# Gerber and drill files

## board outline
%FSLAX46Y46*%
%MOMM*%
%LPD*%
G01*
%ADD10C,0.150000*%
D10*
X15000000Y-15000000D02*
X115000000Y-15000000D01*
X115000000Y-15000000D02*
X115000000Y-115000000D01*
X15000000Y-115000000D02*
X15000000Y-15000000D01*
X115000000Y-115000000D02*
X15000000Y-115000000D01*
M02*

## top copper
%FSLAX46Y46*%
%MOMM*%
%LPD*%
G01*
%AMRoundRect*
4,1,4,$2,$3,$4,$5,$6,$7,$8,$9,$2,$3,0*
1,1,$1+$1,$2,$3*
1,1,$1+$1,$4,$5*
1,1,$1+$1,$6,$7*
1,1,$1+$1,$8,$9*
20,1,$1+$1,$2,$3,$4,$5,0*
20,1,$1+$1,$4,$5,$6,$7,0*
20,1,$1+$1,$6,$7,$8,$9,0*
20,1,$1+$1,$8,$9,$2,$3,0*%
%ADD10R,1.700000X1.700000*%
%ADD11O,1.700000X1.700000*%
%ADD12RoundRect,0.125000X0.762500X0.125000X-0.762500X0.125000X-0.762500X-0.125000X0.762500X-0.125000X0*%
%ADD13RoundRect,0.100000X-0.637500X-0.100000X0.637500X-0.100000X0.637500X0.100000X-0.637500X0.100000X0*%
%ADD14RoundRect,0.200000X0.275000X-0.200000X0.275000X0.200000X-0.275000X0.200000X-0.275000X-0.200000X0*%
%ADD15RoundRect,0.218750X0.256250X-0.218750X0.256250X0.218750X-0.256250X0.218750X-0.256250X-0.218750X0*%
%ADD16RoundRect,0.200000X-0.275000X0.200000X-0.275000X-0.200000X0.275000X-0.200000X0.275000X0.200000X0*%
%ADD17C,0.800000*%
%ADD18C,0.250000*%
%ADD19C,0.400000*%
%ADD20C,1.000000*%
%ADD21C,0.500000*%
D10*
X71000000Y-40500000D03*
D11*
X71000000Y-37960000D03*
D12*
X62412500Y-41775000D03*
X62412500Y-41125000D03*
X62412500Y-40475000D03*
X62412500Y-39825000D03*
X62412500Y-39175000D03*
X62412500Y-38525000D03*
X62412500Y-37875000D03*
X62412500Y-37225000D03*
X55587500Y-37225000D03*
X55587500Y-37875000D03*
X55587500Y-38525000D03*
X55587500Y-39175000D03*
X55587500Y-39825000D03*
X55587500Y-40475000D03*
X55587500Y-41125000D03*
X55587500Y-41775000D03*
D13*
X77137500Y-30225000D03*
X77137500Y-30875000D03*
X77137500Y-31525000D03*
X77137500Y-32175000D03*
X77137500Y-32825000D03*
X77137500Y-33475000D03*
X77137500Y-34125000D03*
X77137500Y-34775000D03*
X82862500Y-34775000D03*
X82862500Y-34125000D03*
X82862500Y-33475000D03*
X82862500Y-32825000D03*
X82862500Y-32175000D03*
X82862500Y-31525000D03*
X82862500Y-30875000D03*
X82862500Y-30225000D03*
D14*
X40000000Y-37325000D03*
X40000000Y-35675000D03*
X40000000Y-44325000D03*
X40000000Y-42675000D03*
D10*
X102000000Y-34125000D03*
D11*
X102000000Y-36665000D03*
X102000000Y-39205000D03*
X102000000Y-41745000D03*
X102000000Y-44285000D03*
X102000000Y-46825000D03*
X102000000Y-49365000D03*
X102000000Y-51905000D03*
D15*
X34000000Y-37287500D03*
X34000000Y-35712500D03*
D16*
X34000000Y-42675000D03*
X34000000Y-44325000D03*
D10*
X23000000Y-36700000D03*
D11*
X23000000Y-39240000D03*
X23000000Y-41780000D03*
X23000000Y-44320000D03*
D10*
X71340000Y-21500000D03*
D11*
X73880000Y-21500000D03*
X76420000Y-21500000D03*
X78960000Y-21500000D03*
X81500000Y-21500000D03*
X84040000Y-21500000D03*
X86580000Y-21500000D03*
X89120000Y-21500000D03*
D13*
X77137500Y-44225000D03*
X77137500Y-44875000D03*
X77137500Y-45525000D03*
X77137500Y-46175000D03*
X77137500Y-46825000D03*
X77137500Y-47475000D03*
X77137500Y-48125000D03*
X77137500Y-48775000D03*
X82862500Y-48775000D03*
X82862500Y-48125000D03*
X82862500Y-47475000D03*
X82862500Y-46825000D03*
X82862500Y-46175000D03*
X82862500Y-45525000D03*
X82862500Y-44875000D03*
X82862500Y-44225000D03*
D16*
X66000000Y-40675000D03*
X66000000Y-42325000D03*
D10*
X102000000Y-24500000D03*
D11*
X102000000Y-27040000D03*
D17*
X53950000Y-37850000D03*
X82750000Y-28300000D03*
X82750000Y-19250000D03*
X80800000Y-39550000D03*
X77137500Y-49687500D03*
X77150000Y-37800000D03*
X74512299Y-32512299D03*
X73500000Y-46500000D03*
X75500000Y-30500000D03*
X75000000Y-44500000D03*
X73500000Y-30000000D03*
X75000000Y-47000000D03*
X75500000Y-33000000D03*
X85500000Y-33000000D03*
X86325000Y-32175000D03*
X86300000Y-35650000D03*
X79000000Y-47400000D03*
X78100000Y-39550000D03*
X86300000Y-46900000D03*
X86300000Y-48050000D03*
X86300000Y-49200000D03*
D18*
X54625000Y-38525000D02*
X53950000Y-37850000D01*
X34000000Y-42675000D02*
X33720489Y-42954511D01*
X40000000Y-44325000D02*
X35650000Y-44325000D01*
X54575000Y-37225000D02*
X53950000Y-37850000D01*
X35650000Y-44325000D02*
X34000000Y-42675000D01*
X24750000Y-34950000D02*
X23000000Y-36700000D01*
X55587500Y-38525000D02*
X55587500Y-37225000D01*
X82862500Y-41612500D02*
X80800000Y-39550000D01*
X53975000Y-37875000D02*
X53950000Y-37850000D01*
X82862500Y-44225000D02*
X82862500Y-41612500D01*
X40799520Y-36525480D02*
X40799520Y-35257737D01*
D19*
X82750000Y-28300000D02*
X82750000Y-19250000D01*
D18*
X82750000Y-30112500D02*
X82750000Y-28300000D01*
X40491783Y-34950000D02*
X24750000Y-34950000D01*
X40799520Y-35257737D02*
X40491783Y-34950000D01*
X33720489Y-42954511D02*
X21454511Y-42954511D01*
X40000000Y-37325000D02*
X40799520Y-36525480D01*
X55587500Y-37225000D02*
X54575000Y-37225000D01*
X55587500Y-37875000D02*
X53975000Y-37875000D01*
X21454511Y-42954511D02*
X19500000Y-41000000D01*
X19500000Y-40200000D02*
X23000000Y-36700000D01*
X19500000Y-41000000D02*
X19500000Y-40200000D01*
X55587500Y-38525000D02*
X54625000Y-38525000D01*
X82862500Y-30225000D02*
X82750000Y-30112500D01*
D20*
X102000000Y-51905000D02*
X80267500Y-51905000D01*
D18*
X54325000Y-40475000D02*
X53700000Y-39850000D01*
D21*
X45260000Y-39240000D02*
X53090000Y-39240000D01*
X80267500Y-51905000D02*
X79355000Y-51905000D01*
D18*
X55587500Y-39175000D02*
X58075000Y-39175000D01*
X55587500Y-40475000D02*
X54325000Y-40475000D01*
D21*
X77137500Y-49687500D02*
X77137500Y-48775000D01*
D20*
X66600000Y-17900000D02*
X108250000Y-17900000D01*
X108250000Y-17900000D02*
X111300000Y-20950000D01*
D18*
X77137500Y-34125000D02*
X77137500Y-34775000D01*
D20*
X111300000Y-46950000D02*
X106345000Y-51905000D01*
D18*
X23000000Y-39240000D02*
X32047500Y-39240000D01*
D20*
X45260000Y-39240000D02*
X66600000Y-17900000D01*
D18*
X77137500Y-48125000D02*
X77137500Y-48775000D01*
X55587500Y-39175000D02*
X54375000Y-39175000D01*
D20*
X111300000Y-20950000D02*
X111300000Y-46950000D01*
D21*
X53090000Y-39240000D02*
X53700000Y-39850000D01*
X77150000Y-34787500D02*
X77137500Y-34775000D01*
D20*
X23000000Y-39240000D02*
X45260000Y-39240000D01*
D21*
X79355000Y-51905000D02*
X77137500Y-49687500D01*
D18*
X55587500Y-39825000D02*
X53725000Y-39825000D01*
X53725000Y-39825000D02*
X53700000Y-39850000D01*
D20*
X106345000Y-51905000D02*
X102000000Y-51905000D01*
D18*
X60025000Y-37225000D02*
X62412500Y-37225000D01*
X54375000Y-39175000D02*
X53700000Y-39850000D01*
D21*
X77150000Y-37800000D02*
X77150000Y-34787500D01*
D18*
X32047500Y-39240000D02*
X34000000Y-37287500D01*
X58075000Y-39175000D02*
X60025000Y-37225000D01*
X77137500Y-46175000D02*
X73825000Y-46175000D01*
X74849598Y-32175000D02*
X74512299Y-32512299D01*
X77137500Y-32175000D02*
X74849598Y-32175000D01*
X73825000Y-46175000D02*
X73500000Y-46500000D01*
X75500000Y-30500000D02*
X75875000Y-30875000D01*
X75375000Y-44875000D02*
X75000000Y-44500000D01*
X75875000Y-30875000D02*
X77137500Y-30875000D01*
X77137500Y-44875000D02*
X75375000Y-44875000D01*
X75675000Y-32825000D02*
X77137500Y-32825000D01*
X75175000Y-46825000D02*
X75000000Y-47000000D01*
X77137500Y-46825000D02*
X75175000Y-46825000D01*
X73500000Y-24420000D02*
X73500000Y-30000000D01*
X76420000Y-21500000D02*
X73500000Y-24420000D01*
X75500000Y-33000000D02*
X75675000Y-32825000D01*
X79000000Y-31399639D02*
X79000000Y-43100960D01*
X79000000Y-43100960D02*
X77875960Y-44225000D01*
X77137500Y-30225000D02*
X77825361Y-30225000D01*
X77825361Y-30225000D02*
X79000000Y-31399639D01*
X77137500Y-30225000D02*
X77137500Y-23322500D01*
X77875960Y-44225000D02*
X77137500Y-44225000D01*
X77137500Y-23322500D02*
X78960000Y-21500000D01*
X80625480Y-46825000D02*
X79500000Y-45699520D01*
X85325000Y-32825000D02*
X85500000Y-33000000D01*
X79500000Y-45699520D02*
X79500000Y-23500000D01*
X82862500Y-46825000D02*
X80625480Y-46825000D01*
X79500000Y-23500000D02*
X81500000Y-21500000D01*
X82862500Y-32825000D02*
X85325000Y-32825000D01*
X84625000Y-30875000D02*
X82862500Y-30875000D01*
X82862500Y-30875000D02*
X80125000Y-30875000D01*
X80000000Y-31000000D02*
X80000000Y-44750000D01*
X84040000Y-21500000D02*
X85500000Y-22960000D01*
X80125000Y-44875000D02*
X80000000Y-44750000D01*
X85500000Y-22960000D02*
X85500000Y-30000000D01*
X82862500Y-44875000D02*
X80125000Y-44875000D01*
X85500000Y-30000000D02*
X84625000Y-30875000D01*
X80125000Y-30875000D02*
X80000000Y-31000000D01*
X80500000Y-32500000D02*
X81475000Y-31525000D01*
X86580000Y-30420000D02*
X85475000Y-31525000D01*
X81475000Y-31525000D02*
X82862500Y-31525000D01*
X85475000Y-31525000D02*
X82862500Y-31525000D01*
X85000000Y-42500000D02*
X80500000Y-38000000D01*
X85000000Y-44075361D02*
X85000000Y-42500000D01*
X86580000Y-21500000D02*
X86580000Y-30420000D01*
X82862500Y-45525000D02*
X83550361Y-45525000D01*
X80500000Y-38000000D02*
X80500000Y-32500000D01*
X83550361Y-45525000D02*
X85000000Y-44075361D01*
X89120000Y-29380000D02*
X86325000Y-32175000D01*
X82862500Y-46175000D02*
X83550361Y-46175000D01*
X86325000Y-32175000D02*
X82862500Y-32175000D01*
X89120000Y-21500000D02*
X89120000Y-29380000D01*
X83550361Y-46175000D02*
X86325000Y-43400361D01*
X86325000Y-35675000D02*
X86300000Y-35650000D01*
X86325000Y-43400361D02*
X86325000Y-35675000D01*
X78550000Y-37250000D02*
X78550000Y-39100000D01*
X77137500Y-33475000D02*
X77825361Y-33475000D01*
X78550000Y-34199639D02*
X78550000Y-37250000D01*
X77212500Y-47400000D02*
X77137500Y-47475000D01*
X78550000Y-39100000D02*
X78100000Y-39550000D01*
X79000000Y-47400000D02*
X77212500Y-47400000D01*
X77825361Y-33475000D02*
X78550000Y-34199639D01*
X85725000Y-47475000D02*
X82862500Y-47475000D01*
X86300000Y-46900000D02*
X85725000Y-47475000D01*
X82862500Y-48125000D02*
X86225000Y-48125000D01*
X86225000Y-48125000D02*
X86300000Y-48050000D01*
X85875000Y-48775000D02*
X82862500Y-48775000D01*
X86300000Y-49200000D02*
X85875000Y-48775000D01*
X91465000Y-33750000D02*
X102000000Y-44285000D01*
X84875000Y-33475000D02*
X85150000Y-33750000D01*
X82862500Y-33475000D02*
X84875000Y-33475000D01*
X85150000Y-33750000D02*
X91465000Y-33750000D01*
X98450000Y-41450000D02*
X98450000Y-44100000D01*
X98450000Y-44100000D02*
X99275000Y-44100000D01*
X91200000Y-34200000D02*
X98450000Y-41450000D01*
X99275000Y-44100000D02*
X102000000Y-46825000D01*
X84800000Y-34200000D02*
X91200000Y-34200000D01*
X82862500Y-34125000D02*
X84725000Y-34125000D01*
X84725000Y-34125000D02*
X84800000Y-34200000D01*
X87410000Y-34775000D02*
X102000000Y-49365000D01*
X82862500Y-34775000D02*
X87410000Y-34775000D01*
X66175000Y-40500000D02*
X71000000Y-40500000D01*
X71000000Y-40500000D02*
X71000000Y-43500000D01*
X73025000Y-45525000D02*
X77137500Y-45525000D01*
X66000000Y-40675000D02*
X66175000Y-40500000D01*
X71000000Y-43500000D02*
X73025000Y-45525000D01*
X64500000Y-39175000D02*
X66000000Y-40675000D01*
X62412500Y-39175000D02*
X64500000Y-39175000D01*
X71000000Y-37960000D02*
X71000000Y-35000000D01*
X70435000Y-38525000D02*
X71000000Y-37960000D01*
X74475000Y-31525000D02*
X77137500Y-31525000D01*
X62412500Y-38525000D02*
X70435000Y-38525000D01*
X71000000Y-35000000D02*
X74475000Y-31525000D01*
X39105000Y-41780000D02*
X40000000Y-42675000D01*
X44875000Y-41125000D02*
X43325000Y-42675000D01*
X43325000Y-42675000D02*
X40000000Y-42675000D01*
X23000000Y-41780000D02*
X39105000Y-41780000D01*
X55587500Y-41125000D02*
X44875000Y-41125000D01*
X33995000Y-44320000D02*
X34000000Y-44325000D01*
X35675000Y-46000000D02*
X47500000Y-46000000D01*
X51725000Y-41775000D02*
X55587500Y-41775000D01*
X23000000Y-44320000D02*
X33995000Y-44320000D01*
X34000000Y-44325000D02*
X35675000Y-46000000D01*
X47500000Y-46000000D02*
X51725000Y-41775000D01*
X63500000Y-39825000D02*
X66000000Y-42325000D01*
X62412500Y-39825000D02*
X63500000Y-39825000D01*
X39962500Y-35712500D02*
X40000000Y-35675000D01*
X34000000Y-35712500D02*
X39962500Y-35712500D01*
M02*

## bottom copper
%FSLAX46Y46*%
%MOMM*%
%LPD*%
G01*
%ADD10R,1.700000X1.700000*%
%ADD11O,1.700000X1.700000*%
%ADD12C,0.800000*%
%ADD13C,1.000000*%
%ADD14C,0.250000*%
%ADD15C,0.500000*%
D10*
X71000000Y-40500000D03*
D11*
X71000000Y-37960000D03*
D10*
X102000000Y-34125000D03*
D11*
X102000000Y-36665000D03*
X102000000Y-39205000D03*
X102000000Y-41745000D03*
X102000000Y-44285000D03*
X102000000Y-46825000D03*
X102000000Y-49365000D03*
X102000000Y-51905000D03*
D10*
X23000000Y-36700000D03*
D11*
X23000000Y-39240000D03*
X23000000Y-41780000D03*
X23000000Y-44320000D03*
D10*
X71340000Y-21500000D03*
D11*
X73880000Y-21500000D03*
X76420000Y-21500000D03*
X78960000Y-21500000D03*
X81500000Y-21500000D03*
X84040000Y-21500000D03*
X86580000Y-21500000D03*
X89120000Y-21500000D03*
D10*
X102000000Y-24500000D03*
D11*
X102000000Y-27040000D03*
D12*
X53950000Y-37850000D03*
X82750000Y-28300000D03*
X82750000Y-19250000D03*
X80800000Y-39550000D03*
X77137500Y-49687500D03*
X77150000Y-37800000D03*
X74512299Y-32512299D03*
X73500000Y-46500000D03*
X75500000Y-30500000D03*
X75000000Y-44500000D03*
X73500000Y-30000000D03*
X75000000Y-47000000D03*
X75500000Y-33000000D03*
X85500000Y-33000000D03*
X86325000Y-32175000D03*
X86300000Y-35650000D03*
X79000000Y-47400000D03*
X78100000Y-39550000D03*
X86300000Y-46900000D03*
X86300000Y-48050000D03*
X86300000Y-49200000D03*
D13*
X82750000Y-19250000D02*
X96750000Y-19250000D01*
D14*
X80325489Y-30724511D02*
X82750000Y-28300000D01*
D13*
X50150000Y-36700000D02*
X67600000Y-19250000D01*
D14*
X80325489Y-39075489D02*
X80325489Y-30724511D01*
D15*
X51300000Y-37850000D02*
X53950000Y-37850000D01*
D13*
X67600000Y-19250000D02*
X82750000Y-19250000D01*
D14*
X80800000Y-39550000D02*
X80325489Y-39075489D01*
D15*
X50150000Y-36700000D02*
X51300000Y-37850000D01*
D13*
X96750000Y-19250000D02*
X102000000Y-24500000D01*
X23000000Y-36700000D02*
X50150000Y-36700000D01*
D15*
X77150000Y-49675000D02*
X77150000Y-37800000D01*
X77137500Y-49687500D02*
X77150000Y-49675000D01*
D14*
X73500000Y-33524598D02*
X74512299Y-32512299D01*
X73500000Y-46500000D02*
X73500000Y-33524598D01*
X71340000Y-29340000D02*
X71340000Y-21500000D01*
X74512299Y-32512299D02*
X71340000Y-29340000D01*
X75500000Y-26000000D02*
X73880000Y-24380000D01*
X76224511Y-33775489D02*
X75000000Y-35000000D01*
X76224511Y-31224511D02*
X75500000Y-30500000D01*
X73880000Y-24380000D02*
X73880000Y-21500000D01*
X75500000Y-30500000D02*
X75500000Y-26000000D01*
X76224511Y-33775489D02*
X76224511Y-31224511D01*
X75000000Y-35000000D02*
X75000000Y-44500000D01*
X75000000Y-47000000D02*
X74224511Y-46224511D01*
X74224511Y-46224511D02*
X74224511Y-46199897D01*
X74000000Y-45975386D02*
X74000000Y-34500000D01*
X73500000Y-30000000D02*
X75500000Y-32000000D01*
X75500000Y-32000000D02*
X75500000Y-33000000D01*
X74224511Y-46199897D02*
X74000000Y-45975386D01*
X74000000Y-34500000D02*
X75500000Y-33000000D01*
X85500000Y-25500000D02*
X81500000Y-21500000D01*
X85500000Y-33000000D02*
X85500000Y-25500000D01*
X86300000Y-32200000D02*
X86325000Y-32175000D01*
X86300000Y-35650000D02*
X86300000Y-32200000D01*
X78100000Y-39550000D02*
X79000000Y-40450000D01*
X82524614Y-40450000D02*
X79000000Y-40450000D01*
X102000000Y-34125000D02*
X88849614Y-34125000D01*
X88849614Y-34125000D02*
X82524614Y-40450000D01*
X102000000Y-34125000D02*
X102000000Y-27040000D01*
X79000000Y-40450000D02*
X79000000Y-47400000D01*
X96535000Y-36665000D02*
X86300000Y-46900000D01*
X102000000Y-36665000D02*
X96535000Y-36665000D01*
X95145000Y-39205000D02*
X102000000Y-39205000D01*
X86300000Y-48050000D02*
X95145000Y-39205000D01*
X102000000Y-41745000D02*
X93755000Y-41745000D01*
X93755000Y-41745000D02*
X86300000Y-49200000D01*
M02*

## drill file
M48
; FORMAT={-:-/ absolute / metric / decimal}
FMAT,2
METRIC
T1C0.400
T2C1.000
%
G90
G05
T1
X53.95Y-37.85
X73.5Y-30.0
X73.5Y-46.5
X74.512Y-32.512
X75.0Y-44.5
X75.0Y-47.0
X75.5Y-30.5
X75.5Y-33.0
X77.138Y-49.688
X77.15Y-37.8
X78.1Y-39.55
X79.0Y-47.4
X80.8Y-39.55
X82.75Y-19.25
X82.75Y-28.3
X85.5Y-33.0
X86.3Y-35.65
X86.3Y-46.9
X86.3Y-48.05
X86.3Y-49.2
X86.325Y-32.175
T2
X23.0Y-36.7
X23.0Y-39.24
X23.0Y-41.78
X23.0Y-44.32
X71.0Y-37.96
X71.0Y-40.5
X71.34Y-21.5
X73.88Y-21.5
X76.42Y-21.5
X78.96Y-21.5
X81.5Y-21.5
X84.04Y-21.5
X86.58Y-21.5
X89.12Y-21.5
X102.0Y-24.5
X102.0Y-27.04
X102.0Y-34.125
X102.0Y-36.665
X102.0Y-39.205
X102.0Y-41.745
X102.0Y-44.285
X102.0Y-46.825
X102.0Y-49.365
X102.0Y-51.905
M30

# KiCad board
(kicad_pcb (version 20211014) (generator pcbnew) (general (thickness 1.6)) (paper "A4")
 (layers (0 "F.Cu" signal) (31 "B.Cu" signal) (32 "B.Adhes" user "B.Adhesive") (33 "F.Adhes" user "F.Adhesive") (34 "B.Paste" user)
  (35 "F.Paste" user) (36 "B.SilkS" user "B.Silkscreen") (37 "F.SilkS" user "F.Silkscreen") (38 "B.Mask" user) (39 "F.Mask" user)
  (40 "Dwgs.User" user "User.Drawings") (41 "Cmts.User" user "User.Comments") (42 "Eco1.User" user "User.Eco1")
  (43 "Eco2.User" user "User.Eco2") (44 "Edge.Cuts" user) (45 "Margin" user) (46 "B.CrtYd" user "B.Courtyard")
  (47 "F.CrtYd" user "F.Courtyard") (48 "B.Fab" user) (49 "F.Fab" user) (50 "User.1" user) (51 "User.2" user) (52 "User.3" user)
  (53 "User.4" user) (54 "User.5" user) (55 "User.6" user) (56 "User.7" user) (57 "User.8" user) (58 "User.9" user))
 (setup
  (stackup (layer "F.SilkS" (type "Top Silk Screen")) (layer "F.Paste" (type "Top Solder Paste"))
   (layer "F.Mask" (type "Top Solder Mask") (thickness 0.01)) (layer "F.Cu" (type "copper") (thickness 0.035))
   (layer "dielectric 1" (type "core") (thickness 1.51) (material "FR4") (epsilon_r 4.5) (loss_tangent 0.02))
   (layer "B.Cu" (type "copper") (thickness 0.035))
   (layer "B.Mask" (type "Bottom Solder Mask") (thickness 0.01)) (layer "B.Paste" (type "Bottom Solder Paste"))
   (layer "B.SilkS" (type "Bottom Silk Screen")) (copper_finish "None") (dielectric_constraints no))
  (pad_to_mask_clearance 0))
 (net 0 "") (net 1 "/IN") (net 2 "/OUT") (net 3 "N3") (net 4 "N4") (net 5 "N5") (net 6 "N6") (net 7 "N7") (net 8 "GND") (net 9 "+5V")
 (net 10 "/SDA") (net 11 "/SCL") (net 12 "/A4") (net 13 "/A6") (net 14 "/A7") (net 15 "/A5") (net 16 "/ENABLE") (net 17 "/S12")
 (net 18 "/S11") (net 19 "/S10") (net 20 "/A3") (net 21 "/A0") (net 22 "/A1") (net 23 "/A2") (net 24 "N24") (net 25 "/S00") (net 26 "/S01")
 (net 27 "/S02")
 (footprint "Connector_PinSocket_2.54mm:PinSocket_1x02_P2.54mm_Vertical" (layer "F.Cu") (at 71 40.5 180)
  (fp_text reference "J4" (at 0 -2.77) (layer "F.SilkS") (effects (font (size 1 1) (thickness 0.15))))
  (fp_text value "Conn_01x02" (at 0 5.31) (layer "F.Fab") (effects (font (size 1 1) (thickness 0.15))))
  (pad "1" thru_hole rect locked (at 0 0 180) (size 1.7 1.7) (drill 1) (layers *.Cu *.Mask) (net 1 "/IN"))
  (pad "2" thru_hole oval locked (at 0 2.54 180) (size 1.7 1.7) (drill 1) (layers *.Cu *.Mask) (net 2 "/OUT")))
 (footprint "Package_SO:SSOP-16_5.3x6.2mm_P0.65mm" (layer "F.Cu") (at 59 39.5 180)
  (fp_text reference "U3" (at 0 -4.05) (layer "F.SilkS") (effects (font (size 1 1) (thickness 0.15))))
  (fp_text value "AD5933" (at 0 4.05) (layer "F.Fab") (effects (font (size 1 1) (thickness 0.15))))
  (pad "1" smd roundrect locked (at -3.4125 -2.275 180) (size 1.775 0.5) (layers "F.Cu" "F.Paste" "F.Mask") (roundrect_rratio 0.25)
   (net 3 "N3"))
  (pad "2" smd roundrect locked (at -3.4125 -1.625 180) (size 1.775 0.5) (layers "F.Cu" "F.Paste" "F.Mask") (roundrect_rratio 0.25)
   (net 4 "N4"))
  (pad "3" smd roundrect locked (at -3.4125 -0.975 180) (size 1.775 0.5) (layers "F.Cu" "F.Paste" "F.Mask") (roundrect_rratio 0.25)
   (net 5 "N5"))
  (pad "4" smd roundrect locked (at -3.4125 -0.325 180) (size 1.775 0.5) (layers "F.Cu" "F.Paste" "F.Mask") (roundrect_rratio 0.25)
   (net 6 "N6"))
  (pad "5" smd roundrect locked (at -3.4125 0.325 180) (size 1.775 0.5) (layers "F.Cu" "F.Paste" "F.Mask") (roundrect_rratio 0.25)
   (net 1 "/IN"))
  (pad "6" smd roundrect locked (at -3.4125 0.975 180) (size 1.775 0.5) (layers "F.Cu" "F.Paste" "F.Mask") (roundrect_rratio 0.25)
   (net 2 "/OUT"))
  (pad "7" smd roundrect locked (at -3.4125 1.625 180) (size 1.775 0.5) (layers "F.Cu" "F.Paste" "F.Mask") (roundrect_rratio 0.25)
   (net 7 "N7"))
  (pad "8" smd roundrect locked (at -3.4125 2.275 180) (size 1.775 0.5) (layers "F.Cu" "F.Paste" "F.Mask") (roundrect_rratio 0.25)
   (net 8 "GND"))
  (pad "9" smd roundrect locked (at 3.4125 2.275 180) (size 1.775 0.5) (layers "F.Cu" "F.Paste" "F.Mask") (roundrect_rratio 0.25)
   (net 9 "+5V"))
  (pad "10" smd roundrect locked (at 3.4125 1.625 180) (size 1.775 0.5) (layers "F.Cu" "F.Paste" "F.Mask") (roundrect_rratio 0.25)
   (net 9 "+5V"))
  (pad "11" smd roundrect locked (at 3.4125 0.975 180) (size 1.775 0.5) (layers "F.Cu" "F.Paste" "F.Mask") (roundrect_rratio 0.25)
   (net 9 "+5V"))
  (pad "12" smd roundrect locked (at 3.4125 0.325 180) (size 1.775 0.5) (layers "F.Cu" "F.Paste" "F.Mask") (roundrect_rratio 0.25)
   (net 8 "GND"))
  (pad "13" smd roundrect locked (at 3.4125 -0.325 180) (size 1.775 0.5) (layers "F.Cu" "F.Paste" "F.Mask") (roundrect_rratio 0.25)
   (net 8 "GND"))
  (pad "14" smd roundrect locked (at 3.4125 -0.975 180) (size 1.775 0.5) (layers "F.Cu" "F.Paste" "F.Mask") (roundrect_rratio 0.25)
   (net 8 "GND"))
  (pad "15" smd roundrect locked (at 3.4125 -1.625 180) (size 1.775 0.5) (layers "F.Cu" "F.Paste" "F.Mask") (roundrect_rratio 0.25)
   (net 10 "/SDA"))
  (pad "16" smd roundrect locked (at 3.4125 -2.275 180) (size 1.775 0.5) (layers "F.Cu" "F.Paste" "F.Mask") (roundrect_rratio 0.25)
   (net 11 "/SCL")))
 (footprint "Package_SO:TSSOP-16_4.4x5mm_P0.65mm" (layer "F.Cu") (at 80 32.5)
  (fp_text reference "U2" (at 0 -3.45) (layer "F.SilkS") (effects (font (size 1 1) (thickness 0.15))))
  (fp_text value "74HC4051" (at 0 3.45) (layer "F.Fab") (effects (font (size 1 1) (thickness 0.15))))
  (pad "1" smd roundrect locked (at -2.8625 -2.275) (size 1.475 0.4) (layers "F.Cu" "F.Paste" "F.Mask") (roundrect_rratio 0.25)
   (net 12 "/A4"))
  (pad "2" smd roundrect locked (at -2.8625 -1.625) (size 1.475 0.4) (layers "F.Cu" "F.Paste" "F.Mask") (roundrect_rratio 0.25)
   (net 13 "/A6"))
  (pad "3" smd roundrect locked (at -2.8625 -0.975) (size 1.475 0.4) (layers "F.Cu" "F.Paste" "F.Mask") (roundrect_rratio 0.25)
   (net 2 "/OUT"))
  (pad "4" smd roundrect locked (at -2.8625 -0.325) (size 1.475 0.4) (layers "F.Cu" "F.Paste" "F.Mask") (roundrect_rratio 0.25)
   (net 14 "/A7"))
  (pad "5" smd roundrect locked (at -2.8625 0.325) (size 1.475 0.4) (layers "F.Cu" "F.Paste" "F.Mask") (roundrect_rratio 0.25)
   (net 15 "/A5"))
  (pad "6" smd roundrect locked (at -2.8625 0.975) (size 1.475 0.4) (layers "F.Cu" "F.Paste" "F.Mask") (roundrect_rratio 0.25)
   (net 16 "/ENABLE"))
  (pad "7" smd roundrect locked (at -2.8625 1.625) (size 1.475 0.4) (layers "F.Cu" "F.Paste" "F.Mask") (roundrect_rratio 0.25) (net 8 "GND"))
  (pad "8" smd roundrect locked (at -2.8625 2.275) (size 1.475 0.4) (layers "F.Cu" "F.Paste" "F.Mask") (roundrect_rratio 0.25) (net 8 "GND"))
  (pad "9" smd roundrect locked (at 2.8625 2.275) (size 1.475 0.4) (layers "F.Cu" "F.Paste" "F.Mask") (roundrect_rratio 0.25)
   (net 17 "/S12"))
  (pad "10" smd roundrect locked (at 2.8625 1.625) (size 1.475 0.4) (layers "F.Cu" "F.Paste" "F.Mask") (roundrect_rratio 0.25)
   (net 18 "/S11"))
  (pad "11" smd roundrect locked (at 2.8625 0.975) (size 1.475 0.4) (layers "F.Cu" "F.Paste" "F.Mask") (roundrect_rratio 0.25)
   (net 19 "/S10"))
  (pad "12" smd roundrect locked (at 2.8625 0.325) (size 1.475 0.4) (layers "F.Cu" "F.Paste" "F.Mask") (roundrect_rratio 0.25)
   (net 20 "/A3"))
  (pad "13" smd roundrect locked (at 2.8625 -0.325) (size 1.475 0.4) (layers "F.Cu" "F.Paste" "F.Mask") (roundrect_rratio 0.25)
   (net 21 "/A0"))
  (pad "14" smd roundrect locked (at 2.8625 -0.975) (size 1.475 0.4) (layers "F.Cu" "F.Paste" "F.Mask") (roundrect_rratio 0.25)
   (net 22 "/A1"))
  (pad "15" smd roundrect locked (at 2.8625 -1.625) (size 1.475 0.4) (layers "F.Cu" "F.Paste" "F.Mask") (roundrect_rratio 0.25)
   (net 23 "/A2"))
  (pad "16" smd roundrect locked (at 2.8625 -2.275) (size 1.475 0.4) (layers "F.Cu" "F.Paste" "F.Mask") (roundrect_rratio 0.25)
   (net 9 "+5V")))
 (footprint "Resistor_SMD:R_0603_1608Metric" (layer "F.Cu") (at 40 36.5 90)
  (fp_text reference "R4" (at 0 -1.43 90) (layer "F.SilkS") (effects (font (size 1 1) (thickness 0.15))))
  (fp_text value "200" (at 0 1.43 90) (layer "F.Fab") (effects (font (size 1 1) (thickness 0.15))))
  (pad "1" smd roundrect locked (at -0.825 0 90) (size 0.8 0.95) (layers "F.Cu" "F.Paste" "F.Mask") (roundrect_rratio 0.25) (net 9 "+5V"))
  (pad "2" smd roundrect locked (at 0.825 0 90) (size 0.8 0.95) (layers "F.Cu" "F.Paste" "F.Mask") (roundrect_rratio 0.25) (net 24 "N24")))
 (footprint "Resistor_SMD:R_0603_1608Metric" (layer "F.Cu") (at 40 43.5 90)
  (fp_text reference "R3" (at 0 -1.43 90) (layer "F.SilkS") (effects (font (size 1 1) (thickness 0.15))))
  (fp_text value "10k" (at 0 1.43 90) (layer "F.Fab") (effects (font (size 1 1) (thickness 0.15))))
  (pad "1" smd roundrect locked (at -0.825 0 90) (size 0.8 0.95) (layers "F.Cu" "F.Paste" "F.Mask") (roundrect_rratio 0.25) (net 9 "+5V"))
  (pad "2" smd roundrect locked (at 0.825 0 90) (size 0.8 0.95) (layers "F.Cu" "F.Paste" "F.Mask") (roundrect_rratio 0.25) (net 10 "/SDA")))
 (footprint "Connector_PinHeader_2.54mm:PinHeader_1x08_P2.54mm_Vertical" (layer "F.Cu") (at 102 34.125)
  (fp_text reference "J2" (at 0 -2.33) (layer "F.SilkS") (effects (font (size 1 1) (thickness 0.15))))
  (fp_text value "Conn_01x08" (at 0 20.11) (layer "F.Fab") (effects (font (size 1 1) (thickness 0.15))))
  (pad "1" thru_hole rect locked (at 0 0) (size 1.7 1.7) (drill 1) (layers *.Cu *.Mask) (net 16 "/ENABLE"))
  (pad "2" thru_hole oval locked (at 0 2.54) (size 1.7 1.7) (drill 1) (layers *.Cu *.Mask) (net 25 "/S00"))
  (pad "3" thru_hole oval locked (at 0 5.08) (size 1.7 1.7) (drill 1) (layers *.Cu *.Mask) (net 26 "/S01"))
  (pad "4" thru_hole oval locked (at 0 7.62) (size 1.7 1.7) (drill 1) (layers *.Cu *.Mask) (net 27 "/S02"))
  (pad "5" thru_hole oval locked (at 0 10.16) (size 1.7 1.7) (drill 1) (layers *.Cu *.Mask) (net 19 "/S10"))
  (pad "6" thru_hole oval locked (at 0 12.7) (size 1.7 1.7) (drill 1) (layers *.Cu *.Mask) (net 18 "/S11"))
  (pad "7" thru_hole oval locked (at 0 15.24) (size 1.7 1.7) (drill 1) (layers *.Cu *.Mask) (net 17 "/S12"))
  (pad "8" thru_hole oval locked (at 0 17.78) (size 1.7 1.7) (drill 1) (layers *.Cu *.Mask) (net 8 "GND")))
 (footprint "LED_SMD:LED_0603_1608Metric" (layer "F.Cu") (at 34 36.5 90)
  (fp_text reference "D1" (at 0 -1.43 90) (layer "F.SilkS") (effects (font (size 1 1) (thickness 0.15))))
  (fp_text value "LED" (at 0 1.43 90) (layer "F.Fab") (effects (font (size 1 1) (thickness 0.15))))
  (pad "1" smd roundrect locked (at -0.7875 0 90) (size 0.875 0.95) (layers "F.Cu" "F.Paste" "F.Mask") (roundrect_rratio 0.25) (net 8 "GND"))
  (pad "2" smd roundrect locked (at 0.7875 0 90) (size 0.875 0.95) (layers "F.Cu" "F.Paste" "F.Mask") (roundrect_rratio 0.25) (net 24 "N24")))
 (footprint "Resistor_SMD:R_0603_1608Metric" (layer "F.Cu") (at 34 43.5 -90)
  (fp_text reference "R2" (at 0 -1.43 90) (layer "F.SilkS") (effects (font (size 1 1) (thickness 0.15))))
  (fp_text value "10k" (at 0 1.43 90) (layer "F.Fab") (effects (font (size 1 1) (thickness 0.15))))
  (pad "1" smd roundrect locked (at -0.825 0 270) (size 0.8 0.95) (layers "F.Cu" "F.Paste" "F.Mask") (roundrect_rratio 0.25) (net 9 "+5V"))
  (pad "2" smd roundrect locked (at 0.825 0 270) (size 0.8 0.95) (layers "F.Cu" "F.Paste" "F.Mask") (roundrect_rratio 0.25) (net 11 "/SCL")))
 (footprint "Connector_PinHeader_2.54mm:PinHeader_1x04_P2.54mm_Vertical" (layer "F.Cu") (at 23 36.7)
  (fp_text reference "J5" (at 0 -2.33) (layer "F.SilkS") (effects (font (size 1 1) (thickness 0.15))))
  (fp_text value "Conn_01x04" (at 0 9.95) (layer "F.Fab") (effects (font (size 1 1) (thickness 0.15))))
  (pad "1" thru_hole rect locked (at 0 0) (size 1.7 1.7) (drill 1) (layers *.Cu *.Mask) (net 9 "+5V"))
  (pad "2" thru_hole oval locked (at 0 2.54) (size 1.7 1.7) (drill 1) (layers *.Cu *.Mask) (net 8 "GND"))
  (pad "3" thru_hole oval locked (at 0 5.08) (size 1.7 1.7) (drill 1) (layers *.Cu *.Mask) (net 10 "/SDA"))
  (pad "4" thru_hole oval locked (at 0 7.62) (size 1.7 1.7) (drill 1) (layers *.Cu *.Mask) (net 11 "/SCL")))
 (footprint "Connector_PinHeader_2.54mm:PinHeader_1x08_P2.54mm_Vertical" (layer "F.Cu") (at 71.34 21.5 90)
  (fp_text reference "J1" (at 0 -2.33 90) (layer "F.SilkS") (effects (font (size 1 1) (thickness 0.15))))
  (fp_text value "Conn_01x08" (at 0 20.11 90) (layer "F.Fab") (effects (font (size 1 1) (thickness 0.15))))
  (pad "1" thru_hole rect locked (at 0 0 90) (size 1.7 1.7) (drill 1) (layers *.Cu *.Mask) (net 14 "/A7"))
  (pad "2" thru_hole oval locked (at 0 2.54 90) (size 1.7 1.7) (drill 1) (layers *.Cu *.Mask) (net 13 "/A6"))
  (pad "3" thru_hole oval locked (at 0 5.08 90) (size 1.7 1.7) (drill 1) (layers *.Cu *.Mask) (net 15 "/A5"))
  (pad "4" thru_hole oval locked (at 0 7.62 90) (size 1.7 1.7) (drill 1) (layers *.Cu *.Mask) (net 12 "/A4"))
  (pad "5" thru_hole oval locked (at 0 10.16 90) (size 1.7 1.7) (drill 1) (layers *.Cu *.Mask) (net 20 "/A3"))
  (pad "6" thru_hole oval locked (at 0 12.7 90) (size 1.7 1.7) (drill 1) (layers *.Cu *.Mask) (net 23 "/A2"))
  (pad "7" thru_hole oval locked (at 0 15.24 90) (size 1.7 1.7) (drill 1) (layers *.Cu *.Mask) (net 22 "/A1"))
  (pad "8" thru_hole oval locked (at 0 17.78 90) (size 1.7 1.7) (drill 1) (layers *.Cu *.Mask) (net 21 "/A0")))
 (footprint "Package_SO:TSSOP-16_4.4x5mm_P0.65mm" (layer "F.Cu") (at 80 46.5)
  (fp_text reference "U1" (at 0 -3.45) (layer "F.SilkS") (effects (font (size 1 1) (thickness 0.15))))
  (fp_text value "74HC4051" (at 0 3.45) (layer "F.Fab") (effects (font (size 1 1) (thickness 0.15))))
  (pad "1" smd roundrect locked (at -2.8625 -2.275) (size 1.475 0.4) (layers "F.Cu" "F.Paste" "F.Mask") (roundrect_rratio 0.25)
   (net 12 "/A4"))
  (pad "2" smd roundrect locked (at -2.8625 -1.625) (size 1.475 0.4) (layers "F.Cu" "F.Paste" "F.Mask") (roundrect_rratio 0.25)
   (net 13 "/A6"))
  (pad "3" smd roundrect locked (at -2.8625 -0.975) (size 1.475 0.4) (layers "F.Cu" "F.Paste" "F.Mask") (roundrect_rratio 0.25)
   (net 1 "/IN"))
  (pad "4" smd roundrect locked (at -2.8625 -0.325) (size 1.475 0.4) (layers "F.Cu" "F.Paste" "F.Mask") (roundrect_rratio 0.25)
   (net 14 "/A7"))
  (pad "5" smd roundrect locked (at -2.8625 0.325) (size 1.475 0.4) (layers "F.Cu" "F.Paste" "F.Mask") (roundrect_rratio 0.25)
   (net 15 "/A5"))
  (pad "6" smd roundrect locked (at -2.8625 0.975) (size 1.475 0.4) (layers "F.Cu" "F.Paste" "F.Mask") (roundrect_rratio 0.25)
   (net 16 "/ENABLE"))
  (pad "7" smd roundrect locked (at -2.8625 1.625) (size 1.475 0.4) (layers "F.Cu" "F.Paste" "F.Mask") (roundrect_rratio 0.25) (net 8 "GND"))
  (pad "8" smd roundrect locked (at -2.8625 2.275) (size 1.475 0.4) (layers "F.Cu" "F.Paste" "F.Mask") (roundrect_rratio 0.25) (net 8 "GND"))
  (pad "9" smd roundrect locked (at 2.8625 2.275) (size 1.475 0.4) (layers "F.Cu" "F.Paste" "F.Mask") (roundrect_rratio 0.25)
   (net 27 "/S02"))
  (pad "10" smd roundrect locked (at 2.8625 1.625) (size 1.475 0.4) (layers "F.Cu" "F.Paste" "F.Mask") (roundrect_rratio 0.25)
   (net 26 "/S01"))
  (pad "11" smd roundrect locked (at 2.8625 0.975) (size 1.475 0.4) (layers "F.Cu" "F.Paste" "F.Mask") (roundrect_rratio 0.25)
   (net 25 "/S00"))
  (pad "12" smd roundrect locked (at 2.8625 0.325) (size 1.475 0.4) (layers "F.Cu" "F.Paste" "F.Mask") (roundrect_rratio 0.25)
   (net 20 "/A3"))
  (pad "13" smd roundrect locked (at 2.8625 -0.325) (size 1.475 0.4) (layers "F.Cu" "F.Paste" "F.Mask") (roundrect_rratio 0.25)
   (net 21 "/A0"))
  (pad "14" smd roundrect locked (at 2.8625 -0.975) (size 1.475 0.4) (layers "F.Cu" "F.Paste" "F.Mask") (roundrect_rratio 0.25)
   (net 22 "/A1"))
  (pad "15" smd roundrect locked (at 2.8625 -1.625) (size 1.475 0.4) (layers "F.Cu" "F.Paste" "F.Mask") (roundrect_rratio 0.25)
   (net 23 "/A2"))
  (pad "16" smd roundrect locked (at 2.8625 -2.275) (size 1.475 0.4) (layers "F.Cu" "F.Paste" "F.Mask") (roundrect_rratio 0.25)
   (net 9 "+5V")))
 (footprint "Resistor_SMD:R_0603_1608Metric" (layer "F.Cu") (at 66 41.5 -90)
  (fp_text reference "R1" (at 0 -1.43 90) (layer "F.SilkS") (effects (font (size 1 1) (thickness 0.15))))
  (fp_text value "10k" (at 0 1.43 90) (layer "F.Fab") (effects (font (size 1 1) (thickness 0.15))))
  (pad "1" smd roundrect locked (at -0.825 0 270) (size 0.8 0.95) (layers "F.Cu" "F.Paste" "F.Mask") (roundrect_rratio 0.25) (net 1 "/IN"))
  (pad "2" smd roundrect locked (at 0.825 0 270) (size 0.8 0.95) (layers "F.Cu" "F.Paste" "F.Mask") (roundrect_rratio 0.25) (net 6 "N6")))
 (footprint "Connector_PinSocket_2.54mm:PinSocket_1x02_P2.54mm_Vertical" (layer "F.Cu") (at 102 24.5)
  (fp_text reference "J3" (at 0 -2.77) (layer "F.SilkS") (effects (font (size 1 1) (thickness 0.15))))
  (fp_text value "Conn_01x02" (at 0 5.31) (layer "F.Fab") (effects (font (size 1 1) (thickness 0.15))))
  (pad "1" thru_hole rect locked (at 0 0) (size 1.7 1.7) (drill 1) (layers *.Cu *.Mask) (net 9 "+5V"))
  (pad "2" thru_hole oval locked (at 0 2.54) (size 1.7 1.7) (drill 1) (layers *.Cu *.Mask) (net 16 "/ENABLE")))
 (gr_line (start 15 15) (end 115 15) (layer "Edge.Cuts") (width 0.15))
 (gr_line (start 115 15) (end 115 115) (layer "Edge.Cuts") (width 0.15))
 (gr_line (start 15 115) (end 15 15) (layer "Edge.Cuts") (width 0.15))
 (gr_line (start 115 115) (end 15 115) (layer "Edge.Cuts") (width 0.15))
 (segment (start 54.625 38.525) (end 53.95 37.85) (width 0.25) (layer "F.Cu") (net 9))
 (segment (start 34 42.675) (end 33.720489 42.954511) (width 0.25) (layer "F.Cu") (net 9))
 (segment (start 40 44.325) (end 35.65 44.325) (width 0.25) (layer "F.Cu") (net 9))
 (segment (start 54.575 37.225) (end 53.95 37.85) (width 0.25) (layer "F.Cu") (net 9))
 (segment (start 35.65 44.325) (end 34 42.675) (width 0.25) (layer "F.Cu") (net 9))
 (segment (start 24.75 34.95) (end 23 36.7) (width 0.25) (layer "F.Cu") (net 9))
 (segment (start 55.5875 38.525) (end 55.5875 37.225) (width 0.25) (layer "F.Cu") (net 9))
 (segment (start 82.8625 41.6125) (end 80.8 39.55) (width 0.25) (layer "F.Cu") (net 9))
 (segment (start 53.975 37.875) (end 53.95 37.85) (width 0.25) (layer "F.Cu") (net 9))
 (segment (start 82.8625 44.225) (end 82.8625 41.6125) (width 0.25) (layer "F.Cu") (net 9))
 (segment (start 40.79952 36.52548) (end 40.79952 35.257737) (width 0.25) (layer "F.Cu") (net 9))
 (segment (start 82.75 28.3) (end 82.75 19.25) (width 0.4) (layer "F.Cu") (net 9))
 (segment (start 82.75 30.1125) (end 82.75 28.3) (width 0.25) (layer "F.Cu") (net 9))
 (segment (start 40.491783 34.95) (end 24.75 34.95) (width 0.25) (layer "F.Cu") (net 9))
 (segment (start 40.79952 35.257737) (end 40.491783 34.95) (width 0.25) (layer "F.Cu") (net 9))
 (segment (start 33.720489 42.954511) (end 21.454511 42.954511) (width 0.25) (layer "F.Cu") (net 9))
 (segment (start 40 37.325) (end 40.79952 36.52548) (width 0.25) (layer "F.Cu") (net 9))
 (segment (start 55.5875 37.225) (end 54.575 37.225) (width 0.25) (layer "F.Cu") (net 9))
 (segment (start 55.5875 37.875) (end 53.975 37.875) (width 0.25) (layer "F.Cu") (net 9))
 (segment (start 21.454511 42.954511) (end 19.5 41) (width 0.25) (layer "F.Cu") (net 9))
 (segment (start 19.5 40.2) (end 23 36.7) (width 0.25) (layer "F.Cu") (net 9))
 (segment (start 19.5 41) (end 19.5 40.2) (width 0.25) (layer "F.Cu") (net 9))
 (segment (start 55.5875 38.525) (end 54.625 38.525) (width 0.25) (layer "F.Cu") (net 9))
 (segment (start 82.8625 30.225) (end 82.75 30.1125) (width 0.25) (layer "F.Cu") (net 9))
 (via (at 53.95 37.85) (size 0.8) (drill 0.4) (layers "F.Cu" "B.Cu") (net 9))
 (via (at 82.75 28.3) (size 0.8) (drill 0.4) (layers "F.Cu" "B.Cu") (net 9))
 (via (at 82.75 19.25) (size 0.8) (drill 0.4) (layers "F.Cu" "B.Cu") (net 9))
 (via (at 80.8 39.55) (size 0.8) (drill 0.4) (layers "F.Cu" "B.Cu") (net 9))
 (segment (start 82.75 19.25) (end 96.75 19.25) (width 1) (layer "B.Cu") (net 9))
 (segment (start 80.325489 30.724511) (end 82.75 28.3) (width 0.25) (layer "B.Cu") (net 9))
 (segment (start 50.15 36.7) (end 67.6 19.25) (width 1) (layer "B.Cu") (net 9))
 (segment (start 80.325489 39.075489) (end 80.325489 30.724511) (width 0.25) (layer "B.Cu") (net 9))
 (segment (start 51.3 37.85) (end 53.95 37.85) (width 0.5) (layer "B.Cu") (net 9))
 (segment (start 67.6 19.25) (end 82.75 19.25) (width 1) (layer "B.Cu") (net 9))
 (segment (start 80.8 39.55) (end 80.325489 39.075489) (width 0.25) (layer "B.Cu") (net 9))
 (segment (start 50.15 36.7) (end 51.3 37.85) (width 0.5) (layer "B.Cu") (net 9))
 (segment (start 96.75 19.25) (end 102 24.5) (width 1) (layer "B.Cu") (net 9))
 (segment (start 23 36.7) (end 50.15 36.7) (width 1) (layer "B.Cu") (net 9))
 (segment (start 102 51.905) (end 80.2675 51.905) (width 1) (layer "F.Cu") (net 8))
 (segment (start 54.325 40.475) (end 53.7 39.85) (width 0.25) (layer "F.Cu") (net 8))
 (segment (start 45.26 39.24) (end 53.09 39.24) (width 0.5) (layer "F.Cu") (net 8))
 (segment (start 80.2675 51.905) (end 79.355 51.905) (width 0.5) (layer "F.Cu") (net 8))
 (segment (start 55.5875 39.175) (end 58.075 39.175) (width 0.25) (layer "F.Cu") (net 8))
 (segment (start 55.5875 40.475) (end 54.325 40.475) (width 0.25) (layer "F.Cu") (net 8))
 (segment (start 77.1375 49.6875) (end 77.1375 48.775) (width 0.5) (layer "F.Cu") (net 8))
 (segment (start 66.6 17.9) (end 108.25 17.9) (width 1) (layer "F.Cu") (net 8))
 (segment (start 108.25 17.9) (end 111.3 20.95) (width 1) (layer "F.Cu") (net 8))
 (segment (start 77.1375 34.125) (end 77.1375 34.775) (width 0.25) (layer "F.Cu") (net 8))
 (segment (start 111.3 46.95) (end 106.345 51.905) (width 1) (layer "F.Cu") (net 8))
 (segment (start 23 39.24) (end 32.0475 39.24) (width 0.25) (layer "F.Cu") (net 8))
 (segment (start 45.26 39.24) (end 66.6 17.9) (width 1) (layer "F.Cu") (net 8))
 (segment (start 77.1375 48.125) (end 77.1375 48.775) (width 0.25) (layer "F.Cu") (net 8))
 (segment (start 55.5875 39.175) (end 54.375 39.175) (width 0.25) (layer "F.Cu") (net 8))
 (segment (start 111.3 20.95) (end 111.3 46.95) (width 1) (layer "F.Cu") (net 8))
 (segment (start 53.09 39.24) (end 53.7 39.85) (width 0.5) (layer "F.Cu") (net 8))
 (segment (start 77.15 34.7875) (end 77.1375 34.775) (width 0.5) (layer "F.Cu") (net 8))
 (segment (start 23 39.24) (end 45.26 39.24) (width 1) (layer "F.Cu") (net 8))
 (segment (start 79.355 51.905) (end 77.1375 49.6875) (width 0.5) (layer "F.Cu") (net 8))
 (segment (start 55.5875 39.825) (end 53.725 39.825) (width 0.25) (layer "F.Cu") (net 8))
 (segment (start 53.725 39.825) (end 53.7 39.85) (width 0.25) (layer "F.Cu") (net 8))
 (segment (start 106.345 51.905) (end 102 51.905) (width 1) (layer "F.Cu") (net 8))
 (segment (start 60.025 37.225) (end 62.4125 37.225) (width 0.25) (layer "F.Cu") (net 8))
 (segment (start 54.375 39.175) (end 53.7 39.85) (width 0.25) (layer "F.Cu") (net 8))
 (segment (start 77.15 37.8) (end 77.15 34.7875) (width 0.5) (layer "F.Cu") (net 8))
 (segment (start 32.0475 39.24) (end 34 37.2875) (width 0.25) (layer "F.Cu") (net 8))
 (segment (start 58.075 39.175) (end 60.025 37.225) (width 0.25) (layer "F.Cu") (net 8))
 (via (at 77.1375 49.6875) (size 0.8) (drill 0.4) (layers "F.Cu" "B.Cu") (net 8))
 (via (at 77.15 37.8) (size 0.8) (drill 0.4) (layers "F.Cu" "B.Cu") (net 8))
 (segment (start 77.15 49.675) (end 77.15 37.8) (width 0.5) (layer "B.Cu") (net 8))
 (segment (start 77.1375 49.6875) (end 77.15 49.675) (width 0.5) (layer "B.Cu") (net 8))
 (segment (start 77.1375 46.175) (end 73.825 46.175) (width 0.25) (layer "F.Cu") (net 14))
 (segment (start 74.849598 32.175) (end 74.512299 32.512299) (width 0.25) (layer "F.Cu") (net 14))
 (segment (start 77.1375 32.175) (end 74.849598 32.175) (width 0.25) (layer "F.Cu") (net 14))
 (segment (start 73.825 46.175) (end 73.5 46.5) (width 0.25) (layer "F.Cu") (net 14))
 (via (at 74.512299 32.512299) (size 0.8) (drill 0.4) (layers "F.Cu" "B.Cu") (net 14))
 (via (at 73.5 46.5) (size 0.8) (drill 0.4) (layers "F.Cu" "B.Cu") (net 14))
 (segment (start 73.5 33.524598) (end 74.512299 32.512299) (width 0.25) (layer "B.Cu") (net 14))
 (segment (start 73.5 46.5) (end 73.5 33.524598) (width 0.25) (layer "B.Cu") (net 14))
 (segment (start 71.34 29.34) (end 71.34 21.5) (width 0.25) (layer "B.Cu") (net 14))
 (segment (start 74.512299 32.512299) (end 71.34 29.34) (width 0.25) (layer "B.Cu") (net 14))
 (segment (start 75.5 30.5) (end 75.875 30.875) (width 0.25) (layer "F.Cu") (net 13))
 (segment (start 75.375 44.875) (end 75 44.5) (width 0.25) (layer "F.Cu") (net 13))
 (segment (start 75.875 30.875) (end 77.1375 30.875) (width 0.25) (layer "F.Cu") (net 13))
 (segment (start 77.1375 44.875) (end 75.375 44.875) (width 0.25) (layer "F.Cu") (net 13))
 (via (at 75.5 30.5) (size 0.8) (drill 0.4) (layers "F.Cu" "B.Cu") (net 13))
 (via (at 75 44.5) (size 0.8) (drill 0.4) (layers "F.Cu" "B.Cu") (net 13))
 (segment (start 75.5 26) (end 73.88 24.38) (width 0.25) (layer "B.Cu") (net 13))
 (segment (start 76.224511 33.775489) (end 75 35) (width 0.25) (layer "B.Cu") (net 13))
 (segment (start 76.224511 31.224511) (end 75.5 30.5) (width 0.25) (layer "B.Cu") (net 13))
 (segment (start 73.88 24.38) (end 73.88 21.5) (width 0.25) (layer "B.Cu") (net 13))
 (segment (start 75.5 30.5) (end 75.5 26) (width 0.25) (layer "B.Cu") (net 13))
 (segment (start 76.224511 33.775489) (end 76.224511 31.224511) (width 0.25) (layer "B.Cu") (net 13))
 (segment (start 75 35) (end 75 44.5) (width 0.25) (layer "B.Cu") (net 13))
 (segment (start 75.675 32.825) (end 77.1375 32.825) (width 0.25) (layer "F.Cu") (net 15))
 (segment (start 75.175 46.825) (end 75 47) (width 0.25) (layer "F.Cu") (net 15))
 (segment (start 77.1375 46.825) (end 75.175 46.825) (width 0.25) (layer "F.Cu") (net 15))
 (segment (start 73.5 24.42) (end 73.5 30) (width 0.25) (layer "F.Cu") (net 15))
 (segment (start 76.42 21.5) (end 73.5 24.42) (width 0.25) (layer "F.Cu") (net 15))
 (segment (start 75.5 33) (end 75.675 32.825) (width 0.25) (layer "F.Cu") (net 15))
 (via (at 73.5 30) (size 0.8) (drill 0.4) (layers "F.Cu" "B.Cu") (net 15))
 (via (at 75 47) (size 0.8) (drill 0.4) (layers "F.Cu" "B.Cu") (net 15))
 (via (at 75.5 33) (size 0.8) (drill 0.4) (layers "F.Cu" "B.Cu") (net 15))
 (segment (start 75 47) (end 74.224511 46.224511) (width 0.25) (layer "B.Cu") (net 15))
 (segment (start 74.224511 46.224511) (end 74.224511 46.199897) (width 0.25) (layer "B.Cu") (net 15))
 (segment (start 74 45.975386) (end 74 34.5) (width 0.25) (layer "B.Cu") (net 15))
 (segment (start 73.5 30) (end 75.5 32) (width 0.25) (layer "B.Cu") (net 15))
 (segment (start 75.5 32) (end 75.5 33) (width 0.25) (layer "B.Cu") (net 15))
 (segment (start 74.224511 46.199897) (end 74 45.975386) (width 0.25) (layer "B.Cu") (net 15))
 (segment (start 74 34.5) (end 75.5 33) (width 0.25) (layer "B.Cu") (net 15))
 (segment (start 79 31.399639) (end 79 43.10096) (width 0.25) (layer "F.Cu") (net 12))
 (segment (start 79 43.10096) (end 77.87596 44.225) (width 0.25) (layer "F.Cu") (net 12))
 (segment (start 77.1375 30.225) (end 77.825361 30.225) (width 0.25) (layer "F.Cu") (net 12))
 (segment (start 77.825361 30.225) (end 79 31.399639) (width 0.25) (layer "F.Cu") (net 12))
 (segment (start 77.1375 30.225) (end 77.1375 23.3225) (width 0.25) (layer "F.Cu") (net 12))
 (segment (start 77.87596 44.225) (end 77.1375 44.225) (width 0.25) (layer "F.Cu") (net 12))
 (segment (start 77.1375 23.3225) (end 78.96 21.5) (width 0.25) (layer "F.Cu") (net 12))
 (segment (start 80.62548 46.825) (end 79.5 45.69952) (width 0.25) (layer "F.Cu") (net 20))
 (segment (start 85.325 32.825) (end 85.5 33) (width 0.25) (layer "F.Cu") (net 20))
 (segment (start 79.5 45.69952) (end 79.5 23.5) (width 0.25) (layer "F.Cu") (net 20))
 (segment (start 82.8625 46.825) (end 80.62548 46.825) (width 0.25) (layer "F.Cu") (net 20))
 (segment (start 79.5 23.5) (end 81.5 21.5) (width 0.25) (layer "F.Cu") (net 20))
 (segment (start 82.8625 32.825) (end 85.325 32.825) (width 0.25) (layer "F.Cu") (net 20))
 (via (at 85.5 33) (size 0.8) (drill 0.4) (layers "F.Cu" "B.Cu") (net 20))
 (segment (start 85.5 25.5) (end 81.5 21.5) (width 0.25) (layer "B.Cu") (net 20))
 (segment (start 85.5 33) (end 85.5 25.5) (width 0.25) (layer "B.Cu") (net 20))
 (segment (start 84.625 30.875) (end 82.8625 30.875) (width 0.25) (layer "F.Cu") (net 23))
 (segment (start 82.8625 30.875) (end 80.125 30.875) (width 0.25) (layer "F.Cu") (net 23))
 (segment (start 80 31) (end 80 44.75) (width 0.25) (layer "F.Cu") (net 23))
 (segment (start 84.04 21.5) (end 85.5 22.96) (width 0.25) (layer "F.Cu") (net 23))
 (segment (start 80.125 44.875) (end 80 44.75) (width 0.25) (layer "F.Cu") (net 23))
 (segment (start 85.5 22.96) (end 85.5 30) (width 0.25) (layer "F.Cu") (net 23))
 (segment (start 82.8625 44.875) (end 80.125 44.875) (width 0.25) (layer "F.Cu") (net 23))
 (segment (start 85.5 30) (end 84.625 30.875) (width 0.25) (layer "F.Cu") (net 23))
 (segment (start 80.125 30.875) (end 80 31) (width 0.25) (layer "F.Cu") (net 23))
 (segment (start 80.5 32.5) (end 81.475 31.525) (width 0.25) (layer "F.Cu") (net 22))
 (segment (start 86.58 30.42) (end 85.475 31.525) (width 0.25) (layer "F.Cu") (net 22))
 (segment (start 81.475 31.525) (end 82.8625 31.525) (width 0.25) (layer "F.Cu") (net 22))
 (segment (start 85.475 31.525) (end 82.8625 31.525) (width 0.25) (layer "F.Cu") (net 22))
 (segment (start 85 42.5) (end 80.5 38) (width 0.25) (layer "F.Cu") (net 22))
 (segment (start 85 44.075361) (end 85 42.5) (width 0.25) (layer "F.Cu") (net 22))
 (segment (start 86.58 21.5) (end 86.58 30.42) (width 0.25) (layer "F.Cu") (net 22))
 (segment (start 82.8625 45.525) (end 83.550361 45.525) (width 0.25) (layer "F.Cu") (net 22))
 (segment (start 80.5 38) (end 80.5 32.5) (width 0.25) (layer "F.Cu") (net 22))
 (segment (start 83.550361 45.525) (end 85 44.075361) (width 0.25) (layer "F.Cu") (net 22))
 (segment (start 89.12 29.38) (end 86.325 32.175) (width 0.25) (layer "F.Cu") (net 21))
 (segment (start 82.8625 46.175) (end 83.550361 46.175) (width 0.25) (layer "F.Cu") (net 21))
 (segment (start 86.325 32.175) (end 82.8625 32.175) (width 0.25) (layer "F.Cu") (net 21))
 (segment (start 89.12 21.5) (end 89.12 29.38) (width 0.25) (layer "F.Cu") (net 21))
 (segment (start 83.550361 46.175) (end 86.325 43.400361) (width 0.25) (layer "F.Cu") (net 21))
 (segment (start 86.325 35.675) (end 86.3 35.65) (width 0.25) (layer "F.Cu") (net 21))
 (segment (start 86.325 43.400361) (end 86.325 35.675) (width 0.25) (layer "F.Cu") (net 21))
 (via (at 86.325 32.175) (size 0.8) (drill 0.4) (layers "F.Cu" "B.Cu") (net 21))
 (via (at 86.3 35.65) (size 0.8) (drill 0.4) (layers "F.Cu" "B.Cu") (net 21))
 (segment (start 86.3 32.2) (end 86.325 32.175) (width 0.25) (layer "B.Cu") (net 21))
 (segment (start 86.3 35.65) (end 86.3 32.2) (width 0.25) (layer "B.Cu") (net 21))
 (segment (start 78.55 37.25) (end 78.55 39.1) (width 0.25) (layer "F.Cu") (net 16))
 (segment (start 77.1375 33.475) (end 77.825361 33.475) (width 0.25) (layer "F.Cu") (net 16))
 (segment (start 78.55 34.199639) (end 78.55 37.25) (width 0.25) (layer "F.Cu") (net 16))
 (segment (start 77.2125 47.4) (end 77.1375 47.475) (width 0.25) (layer "F.Cu") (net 16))
 (segment (start 78.55 39.1) (end 78.1 39.55) (width 0.25) (layer "F.Cu") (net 16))
 (segment (start 79 47.4) (end 77.2125 47.4) (width 0.25) (layer "F.Cu") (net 16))
 (segment (start 77.825361 33.475) (end 78.55 34.199639) (width 0.25) (layer "F.Cu") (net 16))
 (via (at 79 47.4) (size 0.8) (drill 0.4) (layers "F.Cu" "B.Cu") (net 16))
 (via (at 78.1 39.55) (size 0.8) (drill 0.4) (layers "F.Cu" "B.Cu") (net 16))
 (segment (start 78.1 39.55) (end 79 40.45) (width 0.25) (layer "B.Cu") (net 16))
 (segment (start 82.524614 40.45) (end 79 40.45) (width 0.25) (layer "B.Cu") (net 16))
 (segment (start 102 34.125) (end 88.849614 34.125) (width 0.25) (layer "B.Cu") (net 16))
 (segment (start 88.849614 34.125) (end 82.524614 40.45) (width 0.25) (layer "B.Cu") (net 16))
 (segment (start 102 34.125) (end 102 27.04) (width 0.25) (layer "B.Cu") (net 16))
 (segment (start 79 40.45) (end 79 47.4) (width 0.25) (layer "B.Cu") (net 16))
 (segment (start 85.725 47.475) (end 82.8625 47.475) (width 0.25) (layer "F.Cu") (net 25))
 (segment (start 86.3 46.9) (end 85.725 47.475) (width 0.25) (layer "F.Cu") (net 25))
 (via (at 86.3 46.9) (size 0.8) (drill 0.4) (layers "F.Cu" "B.Cu") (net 25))
 (segment (start 96.535 36.665) (end 86.3 46.9) (width 0.25) (layer "B.Cu") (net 25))
 (segment (start 102 36.665) (end 96.535 36.665) (width 0.25) (layer "B.Cu") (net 25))
 (segment (start 82.8625 48.125) (end 86.225 48.125) (width 0.25) (layer "F.Cu") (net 26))
 (segment (start 86.225 48.125) (end 86.3 48.05) (width 0.25) (layer "F.Cu") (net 26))
 (via (at 86.3 48.05) (size 0.8) (drill 0.4) (layers "F.Cu" "B.Cu") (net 26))
 (segment (start 95.145 39.205) (end 102 39.205) (width 0.25) (layer "B.Cu") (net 26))
 (segment (start 86.3 48.05) (end 95.145 39.205) (width 0.25) (layer "B.Cu") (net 26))
 (segment (start 85.875 48.775) (end 82.8625 48.775) (width 0.25) (layer "F.Cu") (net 27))
 (segment (start 86.3 49.2) (end 85.875 48.775) (width 0.25) (layer "F.Cu") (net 27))
 (via (at 86.3 49.2) (size 0.8) (drill 0.4) (layers "F.Cu" "B.Cu") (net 27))
 (segment (start 102 41.745) (end 93.755 41.745) (width 0.25) (layer "B.Cu") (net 27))
 (segment (start 93.755 41.745) (end 86.3 49.2) (width 0.25) (layer "B.Cu") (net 27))
 (segment (start 91.465 33.75) (end 102 44.285) (width 0.25) (layer "F.Cu") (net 19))
 (segment (start 84.875 33.475) (end 85.15 33.75) (width 0.25) (layer "F.Cu") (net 19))
 (segment (start 82.8625 33.475) (end 84.875 33.475) (width 0.25) (layer "F.Cu") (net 19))
 (segment (start 85.15 33.75) (end 91.465 33.75) (width 0.25) (layer "F.Cu") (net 19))
 (segment (start 98.45 41.45) (end 98.45 44.1) (width 0.25) (layer "F.Cu") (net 18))
 (segment (start 98.45 44.1) (end 99.275 44.1) (width 0.25) (layer "F.Cu") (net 18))
 (segment (start 91.2 34.2) (end 98.45 41.45) (width 0.25) (layer "F.Cu") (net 18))
 (segment (start 99.275 44.1) (end 102 46.825) (width 0.25) (layer "F.Cu") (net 18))
 (segment (start 84.8 34.2) (end 91.2 34.2) (width 0.25) (layer "F.Cu") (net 18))
 (segment (start 82.8625 34.125) (end 84.725 34.125) (width 0.25) (layer "F.Cu") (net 18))
 (segment (start 84.725 34.125) (end 84.8 34.2) (width 0.25) (layer "F.Cu") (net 18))
 (segment (start 87.41 34.775) (end 102 49.365) (width 0.25) (layer "F.Cu") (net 17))
 (segment (start 82.8625 34.775) (end 87.41 34.775) (width 0.25) (layer "F.Cu") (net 17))
 (segment (start 66.175 40.5) (end 71 40.5) (width 0.25) (layer "F.Cu") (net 1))
 (segment (start 71 40.5) (end 71 43.5) (width 0.25) (layer "F.Cu") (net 1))
 (segment (start 73.025 45.525) (end 77.1375 45.525) (width 0.25) (layer "F.Cu") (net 1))
 (segment (start 66 40.675) (end 66.175 40.5) (width 0.25) (layer "F.Cu") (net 1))
 (segment (start 71 43.5) (end 73.025 45.525) (width 0.25) (layer "F.Cu") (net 1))
 (segment (start 64.5 39.175) (end 66 40.675) (width 0.25) (layer "F.Cu") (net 1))
 (segment (start 62.4125 39.175) (end 64.5 39.175) (width 0.25) (layer "F.Cu") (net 1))
 (segment (start 71 37.96) (end 71 35) (width 0.25) (layer "F.Cu") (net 2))
 (segment (start 70.435 38.525) (end 71 37.96) (width 0.25) (layer "F.Cu") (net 2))
 (segment (start 74.475 31.525) (end 77.1375 31.525) (width 0.25) (layer "F.Cu") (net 2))
 (segment (start 62.4125 38.525) (end 70.435 38.525) (width 0.25) (layer "F.Cu") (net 2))
 (segment (start 71 35) (end 74.475 31.525) (width 0.25) (layer "F.Cu") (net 2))
 (segment (start 39.105 41.78) (end 40 42.675) (width 0.25) (layer "F.Cu") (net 10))
 (segment (start 44.875 41.125) (end 43.325 42.675) (width 0.25) (layer "F.Cu") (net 10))
 (segment (start 43.325 42.675) (end 40 42.675) (width 0.25) (layer "F.Cu") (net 10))
 (segment (start 23 41.78) (end 39.105 41.78) (width 0.25) (layer "F.Cu") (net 10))
 (segment (start 55.5875 41.125) (end 44.875 41.125) (width 0.25) (layer "F.Cu") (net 10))
 (segment (start 33.995 44.32) (end 34 44.325) (width 0.25) (layer "F.Cu") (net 11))
 (segment (start 35.675 46) (end 47.5 46) (width 0.25) (layer "F.Cu") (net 11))
 (segment (start 51.725 41.775) (end 55.5875 41.775) (width 0.25) (layer "F.Cu") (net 11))
 (segment (start 23 44.32) (end 33.995 44.32) (width 0.25) (layer "F.Cu") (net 11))
 (segment (start 34 44.325) (end 35.675 46) (width 0.25) (layer "F.Cu") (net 11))
 (segment (start 47.5 46) (end 51.725 41.775) (width 0.25) (layer "F.Cu") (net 11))
 (segment (start 63.5 39.825) (end 66 42.325) (width 0.25) (layer "F.Cu") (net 6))
 (segment (start 62.4125 39.825) (end 63.5 39.825) (width 0.25) (layer "F.Cu") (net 6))
 (segment (start 39.9625 35.7125) (end 40 35.675) (width 0.25) (layer "F.Cu") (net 24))
 (segment (start 34 35.7125) (end 39.9625 35.7125) (width 0.25) (layer "F.Cu") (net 24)))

